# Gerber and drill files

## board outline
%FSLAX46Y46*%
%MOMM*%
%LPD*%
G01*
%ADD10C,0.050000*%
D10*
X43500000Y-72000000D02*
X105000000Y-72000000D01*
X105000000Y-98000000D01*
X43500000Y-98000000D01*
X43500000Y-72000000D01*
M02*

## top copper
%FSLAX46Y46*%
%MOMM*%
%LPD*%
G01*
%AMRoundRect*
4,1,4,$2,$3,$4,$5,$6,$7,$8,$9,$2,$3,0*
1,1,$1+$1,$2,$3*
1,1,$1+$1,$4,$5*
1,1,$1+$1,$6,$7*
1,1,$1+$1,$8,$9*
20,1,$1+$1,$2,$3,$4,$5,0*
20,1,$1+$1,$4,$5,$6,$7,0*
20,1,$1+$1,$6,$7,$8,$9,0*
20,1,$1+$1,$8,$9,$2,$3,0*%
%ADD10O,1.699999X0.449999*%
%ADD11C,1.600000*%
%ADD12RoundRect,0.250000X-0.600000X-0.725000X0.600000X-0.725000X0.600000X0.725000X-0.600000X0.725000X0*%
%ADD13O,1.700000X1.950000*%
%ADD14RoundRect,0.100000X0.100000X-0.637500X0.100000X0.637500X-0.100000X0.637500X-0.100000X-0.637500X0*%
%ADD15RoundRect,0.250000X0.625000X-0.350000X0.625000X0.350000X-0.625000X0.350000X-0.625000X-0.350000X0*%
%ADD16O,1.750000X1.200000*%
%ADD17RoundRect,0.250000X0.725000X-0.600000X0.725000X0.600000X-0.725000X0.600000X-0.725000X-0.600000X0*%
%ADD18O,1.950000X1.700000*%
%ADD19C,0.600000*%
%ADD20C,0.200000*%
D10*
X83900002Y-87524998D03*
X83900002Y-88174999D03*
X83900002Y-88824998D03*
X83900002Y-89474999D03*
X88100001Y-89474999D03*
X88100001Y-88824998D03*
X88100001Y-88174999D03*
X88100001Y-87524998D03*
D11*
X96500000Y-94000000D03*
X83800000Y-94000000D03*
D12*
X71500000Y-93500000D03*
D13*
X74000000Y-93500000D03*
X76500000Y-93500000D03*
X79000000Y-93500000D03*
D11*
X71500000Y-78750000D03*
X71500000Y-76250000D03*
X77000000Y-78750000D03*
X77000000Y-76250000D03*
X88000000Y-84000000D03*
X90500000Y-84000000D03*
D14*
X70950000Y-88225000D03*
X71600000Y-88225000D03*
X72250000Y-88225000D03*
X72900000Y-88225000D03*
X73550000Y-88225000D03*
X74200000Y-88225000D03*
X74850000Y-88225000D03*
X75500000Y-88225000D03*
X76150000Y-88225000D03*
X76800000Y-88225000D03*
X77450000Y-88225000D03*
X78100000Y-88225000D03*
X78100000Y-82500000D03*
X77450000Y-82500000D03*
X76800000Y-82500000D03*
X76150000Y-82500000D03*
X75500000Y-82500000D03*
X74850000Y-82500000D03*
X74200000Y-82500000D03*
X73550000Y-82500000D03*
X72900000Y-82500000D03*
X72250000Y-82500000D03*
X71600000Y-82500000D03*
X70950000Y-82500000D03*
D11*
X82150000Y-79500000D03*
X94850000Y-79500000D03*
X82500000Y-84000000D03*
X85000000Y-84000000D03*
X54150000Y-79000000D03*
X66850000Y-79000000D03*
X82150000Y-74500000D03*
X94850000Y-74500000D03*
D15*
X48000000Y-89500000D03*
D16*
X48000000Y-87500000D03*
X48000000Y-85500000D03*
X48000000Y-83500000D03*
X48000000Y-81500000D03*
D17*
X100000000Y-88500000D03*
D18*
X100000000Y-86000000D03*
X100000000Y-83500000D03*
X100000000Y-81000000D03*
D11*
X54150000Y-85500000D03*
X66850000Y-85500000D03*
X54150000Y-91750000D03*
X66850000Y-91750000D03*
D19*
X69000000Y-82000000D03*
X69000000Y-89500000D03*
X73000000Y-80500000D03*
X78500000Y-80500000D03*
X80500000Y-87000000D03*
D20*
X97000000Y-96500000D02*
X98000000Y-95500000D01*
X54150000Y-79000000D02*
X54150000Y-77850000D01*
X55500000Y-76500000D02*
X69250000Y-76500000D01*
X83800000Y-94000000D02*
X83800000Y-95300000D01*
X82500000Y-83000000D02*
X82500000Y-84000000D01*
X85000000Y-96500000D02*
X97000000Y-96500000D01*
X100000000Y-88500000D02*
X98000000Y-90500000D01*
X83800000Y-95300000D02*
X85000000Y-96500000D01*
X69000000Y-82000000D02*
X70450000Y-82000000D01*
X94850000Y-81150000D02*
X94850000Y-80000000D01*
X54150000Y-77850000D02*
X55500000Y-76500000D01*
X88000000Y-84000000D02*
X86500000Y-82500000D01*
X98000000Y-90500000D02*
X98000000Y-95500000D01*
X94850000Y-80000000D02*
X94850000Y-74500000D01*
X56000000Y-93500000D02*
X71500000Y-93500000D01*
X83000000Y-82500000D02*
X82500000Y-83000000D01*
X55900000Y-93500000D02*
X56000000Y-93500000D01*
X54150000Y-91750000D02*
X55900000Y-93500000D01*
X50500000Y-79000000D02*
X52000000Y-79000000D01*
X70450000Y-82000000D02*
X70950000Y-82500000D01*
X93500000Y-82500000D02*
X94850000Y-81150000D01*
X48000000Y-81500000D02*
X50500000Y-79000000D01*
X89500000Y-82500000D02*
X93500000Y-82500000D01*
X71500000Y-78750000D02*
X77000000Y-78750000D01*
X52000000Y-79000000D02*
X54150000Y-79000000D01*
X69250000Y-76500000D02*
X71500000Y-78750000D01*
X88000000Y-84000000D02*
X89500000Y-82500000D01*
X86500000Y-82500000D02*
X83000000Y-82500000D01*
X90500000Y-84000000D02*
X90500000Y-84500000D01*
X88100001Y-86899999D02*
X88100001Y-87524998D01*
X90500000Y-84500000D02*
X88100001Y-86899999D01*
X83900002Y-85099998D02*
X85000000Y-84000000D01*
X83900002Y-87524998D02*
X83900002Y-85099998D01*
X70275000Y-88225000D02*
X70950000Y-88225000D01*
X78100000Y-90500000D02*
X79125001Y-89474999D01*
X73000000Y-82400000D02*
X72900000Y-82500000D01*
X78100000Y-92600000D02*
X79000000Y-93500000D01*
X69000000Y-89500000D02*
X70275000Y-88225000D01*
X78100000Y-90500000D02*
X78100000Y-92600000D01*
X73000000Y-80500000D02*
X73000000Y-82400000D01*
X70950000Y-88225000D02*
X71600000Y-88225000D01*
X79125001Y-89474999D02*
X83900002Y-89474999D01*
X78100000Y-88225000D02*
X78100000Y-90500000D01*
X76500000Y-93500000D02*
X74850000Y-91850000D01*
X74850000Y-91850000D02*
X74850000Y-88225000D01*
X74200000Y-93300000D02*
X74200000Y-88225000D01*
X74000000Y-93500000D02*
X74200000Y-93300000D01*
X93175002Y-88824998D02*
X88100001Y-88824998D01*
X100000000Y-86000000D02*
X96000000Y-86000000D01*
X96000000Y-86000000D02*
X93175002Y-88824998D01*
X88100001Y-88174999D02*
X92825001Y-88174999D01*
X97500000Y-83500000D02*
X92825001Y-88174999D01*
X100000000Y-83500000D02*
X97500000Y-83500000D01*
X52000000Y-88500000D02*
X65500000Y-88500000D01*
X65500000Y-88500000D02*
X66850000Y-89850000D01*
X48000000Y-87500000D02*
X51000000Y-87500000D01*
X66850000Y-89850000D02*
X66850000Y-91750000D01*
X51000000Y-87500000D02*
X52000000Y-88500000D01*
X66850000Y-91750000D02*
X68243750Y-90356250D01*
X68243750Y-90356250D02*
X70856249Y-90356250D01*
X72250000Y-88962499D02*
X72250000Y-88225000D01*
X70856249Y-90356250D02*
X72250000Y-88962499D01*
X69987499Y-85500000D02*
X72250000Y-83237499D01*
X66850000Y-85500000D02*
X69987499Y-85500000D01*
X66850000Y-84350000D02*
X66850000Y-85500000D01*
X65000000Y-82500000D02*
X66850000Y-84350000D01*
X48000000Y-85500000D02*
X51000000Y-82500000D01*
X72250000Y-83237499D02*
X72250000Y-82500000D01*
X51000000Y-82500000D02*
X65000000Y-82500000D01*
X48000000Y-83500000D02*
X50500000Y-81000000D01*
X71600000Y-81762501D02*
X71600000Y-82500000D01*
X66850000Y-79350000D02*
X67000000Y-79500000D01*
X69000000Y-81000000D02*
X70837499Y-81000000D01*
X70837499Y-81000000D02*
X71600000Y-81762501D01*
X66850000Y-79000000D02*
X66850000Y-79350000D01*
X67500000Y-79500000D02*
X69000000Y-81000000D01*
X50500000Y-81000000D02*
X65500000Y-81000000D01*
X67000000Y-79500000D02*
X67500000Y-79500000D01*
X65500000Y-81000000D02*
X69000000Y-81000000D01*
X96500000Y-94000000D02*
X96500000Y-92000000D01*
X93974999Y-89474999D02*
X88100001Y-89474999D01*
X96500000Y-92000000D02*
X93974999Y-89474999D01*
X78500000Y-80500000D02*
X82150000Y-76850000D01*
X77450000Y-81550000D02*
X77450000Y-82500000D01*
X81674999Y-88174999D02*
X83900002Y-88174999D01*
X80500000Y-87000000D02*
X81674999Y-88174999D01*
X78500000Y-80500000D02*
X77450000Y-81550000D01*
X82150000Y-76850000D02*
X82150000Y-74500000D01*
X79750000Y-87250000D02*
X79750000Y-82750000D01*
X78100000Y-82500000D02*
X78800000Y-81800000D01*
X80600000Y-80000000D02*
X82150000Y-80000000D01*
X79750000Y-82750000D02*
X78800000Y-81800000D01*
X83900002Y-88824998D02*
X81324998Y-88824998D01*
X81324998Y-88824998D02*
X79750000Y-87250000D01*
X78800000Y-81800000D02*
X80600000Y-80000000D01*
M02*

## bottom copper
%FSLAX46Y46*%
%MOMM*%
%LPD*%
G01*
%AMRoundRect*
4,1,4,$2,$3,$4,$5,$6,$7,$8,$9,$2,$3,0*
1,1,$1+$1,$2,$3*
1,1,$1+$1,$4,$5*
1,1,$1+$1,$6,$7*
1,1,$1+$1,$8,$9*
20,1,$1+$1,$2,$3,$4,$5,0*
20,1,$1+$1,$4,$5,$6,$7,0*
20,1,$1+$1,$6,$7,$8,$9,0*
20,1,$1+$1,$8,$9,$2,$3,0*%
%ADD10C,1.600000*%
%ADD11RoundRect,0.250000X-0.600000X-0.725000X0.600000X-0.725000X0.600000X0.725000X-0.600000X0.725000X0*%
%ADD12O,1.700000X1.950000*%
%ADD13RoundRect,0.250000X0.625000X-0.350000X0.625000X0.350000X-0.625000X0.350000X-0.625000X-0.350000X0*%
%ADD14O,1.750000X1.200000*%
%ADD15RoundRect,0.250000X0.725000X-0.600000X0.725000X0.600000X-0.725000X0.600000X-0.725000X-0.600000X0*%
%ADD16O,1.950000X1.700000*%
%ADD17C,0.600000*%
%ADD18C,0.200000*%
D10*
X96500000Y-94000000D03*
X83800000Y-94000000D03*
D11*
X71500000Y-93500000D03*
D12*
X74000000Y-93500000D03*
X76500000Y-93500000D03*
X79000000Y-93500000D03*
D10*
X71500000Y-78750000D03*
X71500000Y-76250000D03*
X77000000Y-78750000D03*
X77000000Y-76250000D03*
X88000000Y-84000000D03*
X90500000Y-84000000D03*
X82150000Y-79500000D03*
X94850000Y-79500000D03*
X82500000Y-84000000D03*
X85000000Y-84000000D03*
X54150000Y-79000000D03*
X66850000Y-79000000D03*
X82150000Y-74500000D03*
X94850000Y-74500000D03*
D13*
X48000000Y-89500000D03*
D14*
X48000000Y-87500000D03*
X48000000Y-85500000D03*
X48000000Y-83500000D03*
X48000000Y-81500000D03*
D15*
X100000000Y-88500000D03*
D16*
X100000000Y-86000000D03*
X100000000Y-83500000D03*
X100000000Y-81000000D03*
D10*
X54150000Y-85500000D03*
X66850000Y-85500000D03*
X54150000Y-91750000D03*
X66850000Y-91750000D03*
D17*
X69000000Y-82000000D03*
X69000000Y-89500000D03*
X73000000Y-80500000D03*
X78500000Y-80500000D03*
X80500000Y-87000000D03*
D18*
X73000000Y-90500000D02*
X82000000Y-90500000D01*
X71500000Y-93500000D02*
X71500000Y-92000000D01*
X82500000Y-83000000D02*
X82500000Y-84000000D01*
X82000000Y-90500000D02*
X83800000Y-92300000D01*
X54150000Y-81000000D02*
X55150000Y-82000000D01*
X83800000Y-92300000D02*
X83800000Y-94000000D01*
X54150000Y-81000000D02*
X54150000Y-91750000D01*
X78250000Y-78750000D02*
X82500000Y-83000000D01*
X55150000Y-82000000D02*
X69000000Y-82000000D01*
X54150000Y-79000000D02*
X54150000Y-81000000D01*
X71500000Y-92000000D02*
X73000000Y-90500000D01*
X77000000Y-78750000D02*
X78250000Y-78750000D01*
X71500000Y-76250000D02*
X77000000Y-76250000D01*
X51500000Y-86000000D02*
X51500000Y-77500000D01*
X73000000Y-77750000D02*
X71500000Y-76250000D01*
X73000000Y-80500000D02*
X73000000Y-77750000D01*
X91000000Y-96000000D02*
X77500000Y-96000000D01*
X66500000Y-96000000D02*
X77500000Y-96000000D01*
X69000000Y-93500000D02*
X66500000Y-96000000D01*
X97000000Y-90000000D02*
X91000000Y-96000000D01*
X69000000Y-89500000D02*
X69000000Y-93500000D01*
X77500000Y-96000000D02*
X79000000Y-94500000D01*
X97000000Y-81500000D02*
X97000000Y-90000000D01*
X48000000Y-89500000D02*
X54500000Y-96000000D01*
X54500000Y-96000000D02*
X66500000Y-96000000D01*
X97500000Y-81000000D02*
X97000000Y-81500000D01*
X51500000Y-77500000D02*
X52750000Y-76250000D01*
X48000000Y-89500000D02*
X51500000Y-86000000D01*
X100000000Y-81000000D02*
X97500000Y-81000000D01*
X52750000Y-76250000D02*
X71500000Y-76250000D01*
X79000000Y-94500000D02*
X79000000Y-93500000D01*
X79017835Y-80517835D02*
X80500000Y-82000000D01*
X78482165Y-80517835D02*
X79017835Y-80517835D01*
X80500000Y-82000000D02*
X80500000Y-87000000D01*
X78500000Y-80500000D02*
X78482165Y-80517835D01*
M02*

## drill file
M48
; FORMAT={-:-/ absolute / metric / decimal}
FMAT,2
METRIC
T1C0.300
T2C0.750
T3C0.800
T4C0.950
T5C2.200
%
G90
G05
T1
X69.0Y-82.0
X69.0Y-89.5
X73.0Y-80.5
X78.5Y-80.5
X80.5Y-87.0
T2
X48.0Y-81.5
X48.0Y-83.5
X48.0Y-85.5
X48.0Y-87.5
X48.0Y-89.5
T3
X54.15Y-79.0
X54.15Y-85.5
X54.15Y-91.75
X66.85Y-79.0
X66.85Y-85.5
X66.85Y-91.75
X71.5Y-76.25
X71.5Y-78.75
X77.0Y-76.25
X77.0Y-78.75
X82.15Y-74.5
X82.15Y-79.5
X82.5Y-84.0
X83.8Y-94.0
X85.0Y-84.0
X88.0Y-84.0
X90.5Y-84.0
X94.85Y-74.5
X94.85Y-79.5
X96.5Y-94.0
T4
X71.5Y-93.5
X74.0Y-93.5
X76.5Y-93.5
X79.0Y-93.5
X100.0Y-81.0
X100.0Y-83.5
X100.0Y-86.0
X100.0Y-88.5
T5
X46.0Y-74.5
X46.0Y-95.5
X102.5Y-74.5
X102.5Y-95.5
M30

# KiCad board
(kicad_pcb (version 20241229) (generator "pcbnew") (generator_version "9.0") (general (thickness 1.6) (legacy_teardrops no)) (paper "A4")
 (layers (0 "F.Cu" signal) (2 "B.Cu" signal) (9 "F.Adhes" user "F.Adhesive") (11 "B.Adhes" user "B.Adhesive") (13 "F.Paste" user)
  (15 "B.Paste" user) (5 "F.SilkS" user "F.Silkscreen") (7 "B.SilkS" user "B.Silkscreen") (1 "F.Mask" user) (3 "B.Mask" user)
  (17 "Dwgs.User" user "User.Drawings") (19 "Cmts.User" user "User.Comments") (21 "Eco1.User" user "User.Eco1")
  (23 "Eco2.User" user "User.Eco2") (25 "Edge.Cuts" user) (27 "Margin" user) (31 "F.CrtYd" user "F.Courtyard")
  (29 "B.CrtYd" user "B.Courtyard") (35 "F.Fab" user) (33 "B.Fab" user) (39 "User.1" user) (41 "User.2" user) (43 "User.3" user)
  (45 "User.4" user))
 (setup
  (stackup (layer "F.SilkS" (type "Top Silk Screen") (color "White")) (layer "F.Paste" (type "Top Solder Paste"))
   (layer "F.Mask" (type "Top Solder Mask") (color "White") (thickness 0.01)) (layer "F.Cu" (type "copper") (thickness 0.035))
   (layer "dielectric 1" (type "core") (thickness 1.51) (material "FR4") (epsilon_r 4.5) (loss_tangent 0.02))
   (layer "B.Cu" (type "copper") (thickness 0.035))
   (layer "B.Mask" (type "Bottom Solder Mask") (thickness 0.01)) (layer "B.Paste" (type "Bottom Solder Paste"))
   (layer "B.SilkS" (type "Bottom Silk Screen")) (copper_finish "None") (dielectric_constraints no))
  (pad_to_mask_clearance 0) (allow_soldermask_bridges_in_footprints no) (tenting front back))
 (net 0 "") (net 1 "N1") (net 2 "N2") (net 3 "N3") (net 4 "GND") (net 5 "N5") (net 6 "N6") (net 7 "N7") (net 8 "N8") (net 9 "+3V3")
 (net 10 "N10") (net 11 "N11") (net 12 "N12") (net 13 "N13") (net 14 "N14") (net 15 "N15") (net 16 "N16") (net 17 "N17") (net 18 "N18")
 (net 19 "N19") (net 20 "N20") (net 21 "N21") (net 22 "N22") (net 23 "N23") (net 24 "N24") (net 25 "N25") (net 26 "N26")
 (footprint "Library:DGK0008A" (layer "F.Cu") (at 86 88.5)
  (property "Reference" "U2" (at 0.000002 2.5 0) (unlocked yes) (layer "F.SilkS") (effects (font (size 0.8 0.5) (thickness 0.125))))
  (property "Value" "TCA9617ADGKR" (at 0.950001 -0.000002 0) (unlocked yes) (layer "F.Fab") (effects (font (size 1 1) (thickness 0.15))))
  (pad "1" smd oval (at -2.099998 -0.975002 90) (size 0.449999 1.699999) (layers "F.Cu" "F.Mask" "F.Paste") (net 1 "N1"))
  (pad "2" smd oval (at -2.099998 -0.325001 90) (size 0.449999 1.699999) (layers "F.Cu" "F.Mask" "F.Paste") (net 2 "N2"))
  (pad "3" smd oval (at -2.099998 0.324998 90) (size 0.449999 1.699999) (layers "F.Cu" "F.Mask" "F.Paste") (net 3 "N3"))
  (pad "4" smd oval (at -2.099998 0.974999 90) (size 0.449999 1.699999) (layers "F.Cu" "F.Mask" "F.Paste") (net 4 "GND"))
  (pad "5" smd oval (at 2.100001 0.974999 90) (size 0.449999 1.699999) (layers "F.Cu" "F.Mask" "F.Paste") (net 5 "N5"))
  (pad "6" smd oval (at 2.100001 0.324998 90) (size 0.449999 1.699999) (layers "F.Cu" "F.Mask" "F.Paste") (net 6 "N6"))
  (pad "7" smd oval (at 2.100001 -0.325001 90) (size 0.449999 1.699999) (layers "F.Cu" "F.Mask" "F.Paste") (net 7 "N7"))
  (pad "8" smd oval (at 2.100001 -0.975002 90) (size 0.449999 1.699999) (layers "F.Cu" "F.Mask" "F.Paste") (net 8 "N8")))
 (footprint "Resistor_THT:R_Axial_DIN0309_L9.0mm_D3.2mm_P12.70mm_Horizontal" (layer "F.Cu") (at 96.5 94 180)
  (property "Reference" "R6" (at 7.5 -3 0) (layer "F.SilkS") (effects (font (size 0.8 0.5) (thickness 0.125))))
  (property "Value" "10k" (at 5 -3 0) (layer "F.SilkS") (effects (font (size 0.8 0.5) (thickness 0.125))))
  (pad "1" thru_hole circle (at 0 0 180) (size 1.6 1.6) (drill 0.8) (layers "*.Cu" "*.Mask") (remove_unused_layers no) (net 5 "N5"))
  (pad "2" thru_hole circle (at 12.7 0 180) (size 1.6 1.6) (drill 0.8) (layers "*.Cu" "*.Mask") (remove_unused_layers no) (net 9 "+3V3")))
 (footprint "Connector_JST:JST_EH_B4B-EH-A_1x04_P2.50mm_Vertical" (layer "F.Cu") (at 71.5 93.5)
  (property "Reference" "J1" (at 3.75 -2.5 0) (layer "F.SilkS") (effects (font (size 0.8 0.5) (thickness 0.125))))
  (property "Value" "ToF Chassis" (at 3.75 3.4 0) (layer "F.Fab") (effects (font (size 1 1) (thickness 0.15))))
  (pad "1" thru_hole roundrect (at 0 0) (size 1.7 1.95) (drill 0.95) (layers "*.Cu" "*.Mask") (remove_unused_layers no)
   (roundrect_rratio 0.147059) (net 9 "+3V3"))
  (pad "2" thru_hole oval (at 2.5 0) (size 1.7 1.95) (drill 0.95) (layers "*.Cu" "*.Mask") (remove_unused_layers no) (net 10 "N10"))
  (pad "3" thru_hole oval (at 5 0) (size 1.7 1.95) (drill 0.95) (layers "*.Cu" "*.Mask") (remove_unused_layers no) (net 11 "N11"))
  (pad "4" thru_hole oval (at 7.5 0) (size 1.7 1.95) (drill 0.95) (layers "*.Cu" "*.Mask") (remove_unused_layers no) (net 4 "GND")))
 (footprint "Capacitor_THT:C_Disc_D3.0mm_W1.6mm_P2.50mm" (layer "F.Cu") (at 71.5 78.75 90)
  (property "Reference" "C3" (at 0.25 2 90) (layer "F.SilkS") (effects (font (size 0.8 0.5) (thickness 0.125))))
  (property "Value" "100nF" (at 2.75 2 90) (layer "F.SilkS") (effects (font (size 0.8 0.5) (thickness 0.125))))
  (pad "1" thru_hole circle (at 0 0 90) (size 1.6 1.6) (drill 0.8) (layers "*.Cu" "*.Mask") (remove_unused_layers no) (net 9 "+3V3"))
  (pad "2" thru_hole circle (at 2.5 0 90) (size 1.6 1.6) (drill 0.8) (layers "*.Cu" "*.Mask") (remove_unused_layers no) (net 4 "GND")))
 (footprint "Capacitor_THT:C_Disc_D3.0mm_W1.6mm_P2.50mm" (layer "F.Cu") (at 77 78.75 90)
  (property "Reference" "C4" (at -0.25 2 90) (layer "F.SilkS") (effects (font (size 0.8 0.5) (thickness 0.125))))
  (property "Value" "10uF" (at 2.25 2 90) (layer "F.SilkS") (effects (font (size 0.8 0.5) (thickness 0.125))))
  (pad "1" thru_hole circle (at 0 0 90) (size 1.6 1.6) (drill 0.8) (layers "*.Cu" "*.Mask") (remove_unused_layers no) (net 9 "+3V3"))
  (pad "2" thru_hole circle (at 2.5 0 90) (size 1.6 1.6) (drill 0.8) (layers "*.Cu" "*.Mask") (remove_unused_layers no) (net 4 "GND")))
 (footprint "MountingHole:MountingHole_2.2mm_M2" (layer "F.Cu") (at 102.5 95.5)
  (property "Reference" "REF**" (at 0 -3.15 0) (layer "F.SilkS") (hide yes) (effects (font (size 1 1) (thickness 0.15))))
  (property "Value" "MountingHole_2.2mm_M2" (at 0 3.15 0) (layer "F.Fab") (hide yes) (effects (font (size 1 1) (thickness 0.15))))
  (pad "" np_thru_hole circle (at 0 0) (size 2.2 2.2) (drill 2.2) (layers "*.Cu" "*.Mask")))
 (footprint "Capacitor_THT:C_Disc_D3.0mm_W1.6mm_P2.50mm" (layer "F.Cu") (at 88 84)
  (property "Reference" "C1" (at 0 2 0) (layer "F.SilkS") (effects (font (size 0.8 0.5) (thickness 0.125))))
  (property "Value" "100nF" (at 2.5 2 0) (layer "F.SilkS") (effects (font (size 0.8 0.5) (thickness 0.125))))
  (pad "1" thru_hole circle (at 0 0) (size 1.6 1.6) (drill 0.8) (layers "*.Cu" "*.Mask") (remove_unused_layers no) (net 9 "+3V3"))
  (pad "2" thru_hole circle (at 2.5 0) (size 1.6 1.6) (drill 0.8) (layers "*.Cu" "*.Mask") (remove_unused_layers no) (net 8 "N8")))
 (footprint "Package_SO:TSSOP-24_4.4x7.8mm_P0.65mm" (layer "F.Cu") (at 74.525 85.3625 90)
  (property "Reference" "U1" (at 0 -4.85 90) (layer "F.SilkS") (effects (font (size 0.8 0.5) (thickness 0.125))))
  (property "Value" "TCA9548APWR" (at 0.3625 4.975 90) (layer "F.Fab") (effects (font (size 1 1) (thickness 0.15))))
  (pad "1" smd roundrect (at -2.8625 -3.575 90) (size 1.475 0.4) (layers "F.Cu" "F.Mask" "F.Paste") (roundrect_rratio 0.25) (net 4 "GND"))
  (pad "2" smd roundrect (at -2.8625 -2.925 90) (size 1.475 0.4) (layers "F.Cu" "F.Mask" "F.Paste") (roundrect_rratio 0.25) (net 4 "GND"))
  (pad "3" smd roundrect (at -2.8625 -2.275 90) (size 1.475 0.4) (layers "F.Cu" "F.Mask" "F.Paste") (roundrect_rratio 0.25) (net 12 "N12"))
  (pad "4" smd roundrect (at -2.8625 -1.625 90) (size 1.475 0.4) (layers "F.Cu" "F.Mask" "F.Paste") (roundrect_rratio 0.25) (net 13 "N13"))
  (pad "5" smd roundrect (at -2.8625 -0.975 90) (size 1.475 0.4) (layers "F.Cu" "F.Mask" "F.Paste") (roundrect_rratio 0.25) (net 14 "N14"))
  (pad "6" smd roundrect (at -2.8625 -0.325 90) (size 1.475 0.4) (layers "F.Cu" "F.Mask" "F.Paste") (roundrect_rratio 0.25) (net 10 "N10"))
  (pad "7" smd roundrect (at -2.8625 0.325 90) (size 1.475 0.4) (layers "F.Cu" "F.Mask" "F.Paste") (roundrect_rratio 0.25) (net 11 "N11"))
  (pad "8" smd roundrect (at -2.8625 0.975 90) (size 1.475 0.4) (layers "F.Cu" "F.Mask" "F.Paste") (roundrect_rratio 0.25) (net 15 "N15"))
  (pad "9" smd roundrect (at -2.8625 1.625 90) (size 1.475 0.4) (layers "F.Cu" "F.Mask" "F.Paste") (roundrect_rratio 0.25) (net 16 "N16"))
  (pad "10" smd roundrect (at -2.8625 2.275 90) (size 1.475 0.4) (layers "F.Cu" "F.Mask" "F.Paste") (roundrect_rratio 0.25) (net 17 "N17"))
  (pad "11" smd roundrect (at -2.8625 2.925 90) (size 1.475 0.4) (layers "F.Cu" "F.Mask" "F.Paste") (roundrect_rratio 0.25) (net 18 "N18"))
  (pad "12" smd roundrect (at -2.8625 3.575 90) (size 1.475 0.4) (layers "F.Cu" "F.Mask" "F.Paste") (roundrect_rratio 0.25) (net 4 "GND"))
  (pad "13" smd roundrect (at 2.8625 3.575 90) (size 1.475 0.4) (layers "F.Cu" "F.Mask" "F.Paste") (roundrect_rratio 0.25) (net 3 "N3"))
  (pad "14" smd roundrect (at 2.8625 2.925 90) (size 1.475 0.4) (layers "F.Cu" "F.Mask" "F.Paste") (roundrect_rratio 0.25) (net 2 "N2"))
  (pad "15" smd roundrect (at 2.8625 2.275 90) (size 1.475 0.4) (layers "F.Cu" "F.Mask" "F.Paste") (roundrect_rratio 0.25) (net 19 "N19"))
  (pad "16" smd roundrect (at 2.8625 1.625 90) (size 1.475 0.4) (layers "F.Cu" "F.Mask" "F.Paste") (roundrect_rratio 0.25) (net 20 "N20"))
  (pad "17" smd roundrect (at 2.8625 0.975 90) (size 1.475 0.4) (layers "F.Cu" "F.Mask" "F.Paste") (roundrect_rratio 0.25) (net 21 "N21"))
  (pad "18" smd roundrect (at 2.8625 0.325 90) (size 1.475 0.4) (layers "F.Cu" "F.Mask" "F.Paste") (roundrect_rratio 0.25) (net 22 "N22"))
  (pad "19" smd roundrect (at 2.8625 -0.325 90) (size 1.475 0.4) (layers "F.Cu" "F.Mask" "F.Paste") (roundrect_rratio 0.25) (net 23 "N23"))
  (pad "20" smd roundrect (at 2.8625 -0.975 90) (size 1.475 0.4) (layers "F.Cu" "F.Mask" "F.Paste") (roundrect_rratio 0.25) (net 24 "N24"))
  (pad "21" smd roundrect (at 2.8625 -1.625 90) (size 1.475 0.4) (layers "F.Cu" "F.Mask" "F.Paste") (roundrect_rratio 0.25) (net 4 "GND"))
  (pad "22" smd roundrect (at 2.8625 -2.275 90) (size 1.475 0.4) (layers "F.Cu" "F.Mask" "F.Paste") (roundrect_rratio 0.25) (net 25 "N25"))
  (pad "23" smd roundrect (at 2.8625 -2.925 90) (size 1.475 0.4) (layers "F.Cu" "F.Mask" "F.Paste") (roundrect_rratio 0.25) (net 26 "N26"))
  (pad "24" smd roundrect (at 2.8625 -3.575 90) (size 1.475 0.4) (layers "F.Cu" "F.Mask" "F.Paste") (roundrect_rratio 0.25) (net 9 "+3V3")))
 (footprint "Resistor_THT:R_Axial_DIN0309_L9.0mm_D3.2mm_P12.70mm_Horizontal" (layer "F.Cu") (at 82.15 79.5)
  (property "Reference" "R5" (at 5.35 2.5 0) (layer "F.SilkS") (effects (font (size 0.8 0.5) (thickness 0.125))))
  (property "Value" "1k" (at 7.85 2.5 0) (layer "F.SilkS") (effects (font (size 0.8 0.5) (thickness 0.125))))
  (pad "1" thru_hole circle (at 0 0) (size 1.6 1.6) (drill 0.8) (layers "*.Cu" "*.Mask") (remove_unused_layers no) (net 3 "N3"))
  (pad "2" thru_hole circle (at 12.7 0) (size 1.6 1.6) (drill 0.8) (layers "*.Cu" "*.Mask") (remove_unused_layers no) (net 9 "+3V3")))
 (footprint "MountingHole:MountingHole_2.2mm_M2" (layer "F.Cu") (at 46 74.5)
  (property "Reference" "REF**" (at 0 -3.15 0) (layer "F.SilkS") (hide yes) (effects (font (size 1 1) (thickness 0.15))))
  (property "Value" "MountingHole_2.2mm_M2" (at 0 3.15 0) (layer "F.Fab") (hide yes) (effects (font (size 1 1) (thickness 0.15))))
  (pad "" np_thru_hole circle (at 0 0) (size 2.2 2.2) (drill 2.2) (layers "*.Cu" "*.Mask")))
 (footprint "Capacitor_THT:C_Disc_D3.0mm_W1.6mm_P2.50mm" (layer "F.Cu") (at 82.5 84)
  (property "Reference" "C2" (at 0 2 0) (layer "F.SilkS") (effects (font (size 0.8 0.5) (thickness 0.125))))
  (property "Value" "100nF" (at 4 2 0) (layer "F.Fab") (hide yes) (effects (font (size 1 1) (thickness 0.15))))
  (pad "1" thru_hole circle (at 0 0) (size 1.6 1.6) (drill 0.8) (layers "*.Cu" "*.Mask") (remove_unused_layers no) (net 9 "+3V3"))
  (pad "2" thru_hole circle (at 2.5 0) (size 1.6 1.6) (drill 0.8) (layers "*.Cu" "*.Mask") (remove_unused_layers no) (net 1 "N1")))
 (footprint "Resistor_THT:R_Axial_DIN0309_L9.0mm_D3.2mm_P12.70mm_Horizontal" (layer "F.Cu") (at 54.15 79)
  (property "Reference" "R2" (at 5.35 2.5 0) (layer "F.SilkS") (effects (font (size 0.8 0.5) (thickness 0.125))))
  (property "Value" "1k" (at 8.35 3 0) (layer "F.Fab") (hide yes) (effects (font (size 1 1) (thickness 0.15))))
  (pad "1" thru_hole circle (at 0 0) (size 1.6 1.6) (drill 0.8) (layers "*.Cu" "*.Mask") (remove_unused_layers no) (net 9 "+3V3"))
  (pad "2" thru_hole circle (at 12.7 0) (size 1.6 1.6) (drill 0.8) (layers "*.Cu" "*.Mask") (remove_unused_layers no) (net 26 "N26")))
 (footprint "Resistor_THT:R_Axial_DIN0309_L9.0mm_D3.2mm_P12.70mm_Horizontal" (layer "F.Cu") (at 82.15 74.5)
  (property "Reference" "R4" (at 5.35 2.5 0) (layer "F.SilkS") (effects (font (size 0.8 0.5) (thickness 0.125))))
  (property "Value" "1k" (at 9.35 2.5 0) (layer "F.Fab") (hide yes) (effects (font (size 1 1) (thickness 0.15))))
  (pad "1" thru_hole circle (at 0 0) (size 1.6 1.6) (drill 0.8) (layers "*.Cu" "*.Mask") (remove_unused_layers no) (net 2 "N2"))
  (pad "2" thru_hole circle (at 12.7 0) (size 1.6 1.6) (drill 0.8) (layers "*.Cu" "*.Mask") (remove_unused_layers no) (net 9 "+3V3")))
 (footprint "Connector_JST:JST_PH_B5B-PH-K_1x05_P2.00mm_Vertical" (layer "F.Cu") (at 48 89.5 90)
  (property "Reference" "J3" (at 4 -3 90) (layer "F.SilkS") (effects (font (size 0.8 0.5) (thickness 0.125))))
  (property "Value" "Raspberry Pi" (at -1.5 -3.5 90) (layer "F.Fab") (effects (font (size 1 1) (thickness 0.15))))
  (pad "1" thru_hole roundrect (at 0 0 90) (size 1.2 1.75) (drill 0.75) (layers "*.Cu" "*.Mask") (remove_unused_layers no)
   (roundrect_rratio 0.208333) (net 4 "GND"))
  (pad "2" thru_hole oval (at 2 0 90) (size 1.2 1.75) (drill 0.75) (layers "*.Cu" "*.Mask") (remove_unused_layers no) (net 12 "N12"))
  (pad "3" thru_hole oval (at 4 0 90) (size 1.2 1.75) (drill 0.75) (layers "*.Cu" "*.Mask") (remove_unused_layers no) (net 25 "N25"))
  (pad "4" thru_hole oval (at 6 0 90) (size 1.2 1.75) (drill 0.75) (layers "*.Cu" "*.Mask") (remove_unused_layers no) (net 26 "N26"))
  (pad "5" thru_hole oval (at 8 0 90) (size 1.2 1.75) (drill 0.75) (layers "*.Cu" "*.Mask") (remove_unused_layers no) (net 9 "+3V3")))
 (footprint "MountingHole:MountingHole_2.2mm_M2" (layer "F.Cu") (at 102.5 74.5)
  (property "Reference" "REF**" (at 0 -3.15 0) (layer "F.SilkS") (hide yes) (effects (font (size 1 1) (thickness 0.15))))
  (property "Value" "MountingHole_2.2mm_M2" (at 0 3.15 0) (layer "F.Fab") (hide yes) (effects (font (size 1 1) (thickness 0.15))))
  (pad "" np_thru_hole circle (at 0 0) (size 2.2 2.2) (drill 2.2) (layers "*.Cu" "*.Mask")))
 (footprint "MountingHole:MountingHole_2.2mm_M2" (layer "F.Cu") (at 46 95.5)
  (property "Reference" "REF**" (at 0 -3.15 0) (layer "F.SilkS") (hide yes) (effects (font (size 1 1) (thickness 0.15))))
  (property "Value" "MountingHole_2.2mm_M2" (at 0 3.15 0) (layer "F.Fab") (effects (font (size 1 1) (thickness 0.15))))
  (pad "" np_thru_hole circle (at 0 0) (size 2.2 2.2) (drill 2.2) (layers "*.Cu" "*.Mask")))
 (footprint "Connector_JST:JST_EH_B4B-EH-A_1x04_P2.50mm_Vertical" (layer "F.Cu") (at 100 88.5 90)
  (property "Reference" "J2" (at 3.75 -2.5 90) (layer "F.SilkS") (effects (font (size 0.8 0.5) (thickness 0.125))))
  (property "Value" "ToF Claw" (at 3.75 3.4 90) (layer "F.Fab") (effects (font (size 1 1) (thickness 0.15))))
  (pad "1" thru_hole roundrect (at 0 0 90) (size 1.7 1.95) (drill 0.95) (layers "*.Cu" "*.Mask") (remove_unused_layers no)
   (roundrect_rratio 0.147059) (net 9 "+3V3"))
  (pad "2" thru_hole oval (at 2.5 0 90) (size 1.7 1.95) (drill 0.95) (layers "*.Cu" "*.Mask") (remove_unused_layers no) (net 6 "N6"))
  (pad "3" thru_hole oval (at 5 0 90) (size 1.7 1.95) (drill 0.95) (layers "*.Cu" "*.Mask") (remove_unused_layers no) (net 7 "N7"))
  (pad "4" thru_hole oval (at 7.5 0 90) (size 1.7 1.95) (drill 0.95) (layers "*.Cu" "*.Mask") (remove_unused_layers no) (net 4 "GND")))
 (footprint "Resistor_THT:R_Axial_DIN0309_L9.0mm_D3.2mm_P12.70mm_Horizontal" (layer "F.Cu") (at 54.15 85.5)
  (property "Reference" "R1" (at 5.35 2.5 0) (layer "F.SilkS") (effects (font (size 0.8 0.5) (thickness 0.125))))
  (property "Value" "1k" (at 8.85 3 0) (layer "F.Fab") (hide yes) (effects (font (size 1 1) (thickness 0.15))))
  (pad "1" thru_hole circle (at 0 0) (size 1.6 1.6) (drill 0.8) (layers "*.Cu" "*.Mask") (remove_unused_layers no) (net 9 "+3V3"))
  (pad "2" thru_hole circle (at 12.7 0) (size 1.6 1.6) (drill 0.8) (layers "*.Cu" "*.Mask") (remove_unused_layers no) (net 25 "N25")))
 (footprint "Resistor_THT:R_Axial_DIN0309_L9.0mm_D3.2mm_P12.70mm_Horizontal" (layer "F.Cu") (at 54.15 91.75)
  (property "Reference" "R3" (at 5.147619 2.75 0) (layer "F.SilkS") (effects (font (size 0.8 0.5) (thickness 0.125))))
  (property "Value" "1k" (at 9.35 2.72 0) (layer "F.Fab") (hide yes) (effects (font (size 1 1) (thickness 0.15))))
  (pad "1" thru_hole circle (at 0 0) (size 1.6 1.6) (drill 0.8) (layers "*.Cu" "*.Mask") (remove_unused_layers no) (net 9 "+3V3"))
  (pad "2" thru_hole circle (at 12.7 0) (size 1.6 1.6) (drill 0.8) (layers "*.Cu" "*.Mask") (remove_unused_layers no) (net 12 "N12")))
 (gr_rect (start 43.5 72) (end 105 98) (stroke (width 0.05) (type default)) (fill no) (layer "Edge.Cuts"))
 (segment (start 97 96.5) (end 98 95.5) (width 0.2) (layer "F.Cu") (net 9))
 (segment (start 54.15 79) (end 54.15 77.85) (width 0.2) (layer "F.Cu") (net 9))
 (segment (start 55.5 76.5) (end 69.25 76.5) (width 0.2) (layer "F.Cu") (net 9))
 (segment (start 83.8 94) (end 83.8 95.3) (width 0.2) (layer "F.Cu") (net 9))
 (segment (start 82.5 83) (end 82.5 84) (width 0.2) (layer "F.Cu") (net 9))
 (segment (start 85 96.5) (end 97 96.5) (width 0.2) (layer "F.Cu") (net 9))
 (segment (start 100 88.5) (end 98 90.5) (width 0.2) (layer "F.Cu") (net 9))
 (segment (start 83.8 95.3) (end 85 96.5) (width 0.2) (layer "F.Cu") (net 9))
 (segment (start 69 82) (end 70.45 82) (width 0.2) (layer "F.Cu") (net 9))
 (segment (start 94.85 81.15) (end 94.85 80) (width 0.2) (layer "F.Cu") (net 9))
 (segment (start 54.15 77.85) (end 55.5 76.5) (width 0.2) (layer "F.Cu") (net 9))
 (segment (start 88 84) (end 86.5 82.5) (width 0.2) (layer "F.Cu") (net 9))
 (segment (start 98 90.5) (end 98 95.5) (width 0.2) (layer "F.Cu") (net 9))
 (segment (start 94.85 80) (end 94.85 74.5) (width 0.2) (layer "F.Cu") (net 9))
 (segment (start 56 93.5) (end 71.5 93.5) (width 0.2) (layer "F.Cu") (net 9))
 (segment (start 83 82.5) (end 82.5 83) (width 0.2) (layer "F.Cu") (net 9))
 (segment (start 55.9 93.5) (end 56 93.5) (width 0.2) (layer "F.Cu") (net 9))
 (segment (start 54.15 91.75) (end 55.9 93.5) (width 0.2) (layer "F.Cu") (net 9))
 (segment (start 50.5 79) (end 52 79) (width 0.2) (layer "F.Cu") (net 9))
 (segment (start 70.45 82) (end 70.95 82.5) (width 0.2) (layer "F.Cu") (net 9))
 (segment (start 93.5 82.5) (end 94.85 81.15) (width 0.2) (layer "F.Cu") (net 9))
 (segment (start 48 81.5) (end 50.5 79) (width 0.2) (layer "F.Cu") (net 9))
 (segment (start 89.5 82.5) (end 93.5 82.5) (width 0.2) (layer "F.Cu") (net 9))
 (segment (start 71.5 78.75) (end 77 78.75) (width 0.2) (layer "F.Cu") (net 9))
 (segment (start 52 79) (end 54.15 79) (width 0.2) (layer "F.Cu") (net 9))
 (segment (start 69.25 76.5) (end 71.5 78.75) (width 0.2) (layer "F.Cu") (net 9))
 (segment (start 88 84) (end 89.5 82.5) (width 0.2) (layer "F.Cu") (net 9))
 (segment (start 86.5 82.5) (end 83 82.5) (width 0.2) (layer "F.Cu") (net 9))
 (via (at 69 82) (size 0.6) (drill 0.3) (layers "F.Cu" "B.Cu") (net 9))
 (segment (start 73 90.5) (end 82 90.5) (width 0.2) (layer "B.Cu") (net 9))
 (segment (start 71.5 93.5) (end 71.5 92) (width 0.2) (layer "B.Cu") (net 9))
 (segment (start 82.5 83) (end 82.5 84) (width 0.2) (layer "B.Cu") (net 9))
 (segment (start 82 90.5) (end 83.8 92.3) (width 0.2) (layer "B.Cu") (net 9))
 (segment (start 54.15 81) (end 55.15 82) (width 0.2) (layer "B.Cu") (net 9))
 (segment (start 83.8 92.3) (end 83.8 94) (width 0.2) (layer "B.Cu") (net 9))
 (segment (start 54.15 81) (end 54.15 91.75) (width 0.2) (layer "B.Cu") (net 9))
 (segment (start 78.25 78.75) (end 82.5 83) (width 0.2) (layer "B.Cu") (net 9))
 (segment (start 55.15 82) (end 69 82) (width 0.2) (layer "B.Cu") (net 9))
 (segment (start 54.15 79) (end 54.15 81) (width 0.2) (layer "B.Cu") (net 9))
 (segment (start 71.5 92) (end 73 90.5) (width 0.2) (layer "B.Cu") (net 9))
 (segment (start 77 78.75) (end 78.25 78.75) (width 0.2) (layer "B.Cu") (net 9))
 (segment (start 90.5 84) (end 90.5 84.5) (width 0.2) (layer "F.Cu") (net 8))
 (segment (start 88.100001 86.899999) (end 88.100001 87.524998) (width 0.2) (layer "F.Cu") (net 8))
 (segment (start 90.5 84.5) (end 88.100001 86.899999) (width 0.2) (layer "F.Cu") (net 8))
 (segment (start 83.900002 85.099998) (end 85 84) (width 0.2) (layer "F.Cu") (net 1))
 (segment (start 83.900002 87.524998) (end 83.900002 85.099998) (width 0.2) (layer "F.Cu") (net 1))
 (segment (start 70.275 88.225) (end 70.95 88.225) (width 0.2) (layer "F.Cu") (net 4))
 (segment (start 78.1 90.5) (end 79.125001 89.474999) (width 0.2) (layer "F.Cu") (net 4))
 (segment (start 73 82.4) (end 72.9 82.5) (width 0.2) (layer "F.Cu") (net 4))
 (segment (start 78.1 92.6) (end 79 93.5) (width 0.2) (layer "F.Cu") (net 4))
 (segment (start 69 89.5) (end 70.275 88.225) (width 0.2) (layer "F.Cu") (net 4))
 (segment (start 78.1 90.5) (end 78.1 92.6) (width 0.2) (layer "F.Cu") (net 4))
 (segment (start 73 80.5) (end 73 82.4) (width 0.2) (layer "F.Cu") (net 4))
 (segment (start 70.95 88.225) (end 71.6 88.225) (width 0.2) (layer "F.Cu") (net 4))
 (segment (start 79.125001 89.474999) (end 83.900002 89.474999) (width 0.2) (layer "F.Cu") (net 4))
 (segment (start 78.1 88.225) (end 78.1 90.5) (width 0.2) (layer "F.Cu") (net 4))
 (via (at 69 89.5) (size 0.6) (drill 0.3) (layers "F.Cu" "B.Cu") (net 4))
 (via (at 73 80.5) (size 0.6) (drill 0.3) (layers "F.Cu" "B.Cu") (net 4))
 (segment (start 71.5 76.25) (end 77 76.25) (width 0.2) (layer "B.Cu") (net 4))
 (segment (start 51.5 86) (end 51.5 77.5) (width 0.2) (layer "B.Cu") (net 4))
 (segment (start 73 77.75) (end 71.5 76.25) (width 0.2) (layer "B.Cu") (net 4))
 (segment (start 73 80.5) (end 73 77.75) (width 0.2) (layer "B.Cu") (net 4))
 (segment (start 91 96) (end 77.5 96) (width 0.2) (layer "B.Cu") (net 4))
 (segment (start 66.5 96) (end 77.5 96) (width 0.2) (layer "B.Cu") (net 4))
 (segment (start 69 93.5) (end 66.5 96) (width 0.2) (layer "B.Cu") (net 4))
 (segment (start 97 90) (end 91 96) (width 0.2) (layer "B.Cu") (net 4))
 (segment (start 69 89.5) (end 69 93.5) (width 0.2) (layer "B.Cu") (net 4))
 (segment (start 77.5 96) (end 79 94.5) (width 0.2) (layer "B.Cu") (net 4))
 (segment (start 97 81.5) (end 97 90) (width 0.2) (layer "B.Cu") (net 4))
 (segment (start 48 89.5) (end 54.5 96) (width 0.2) (layer "B.Cu") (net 4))
 (segment (start 54.5 96) (end 66.5 96) (width 0.2) (layer "B.Cu") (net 4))
 (segment (start 97.5 81) (end 97 81.5) (width 0.2) (layer "B.Cu") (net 4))
 (segment (start 51.5 77.5) (end 52.75 76.25) (width 0.2) (layer "B.Cu") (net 4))
 (segment (start 48 89.5) (end 51.5 86) (width 0.2) (layer "B.Cu") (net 4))
 (segment (start 100 81) (end 97.5 81) (width 0.2) (layer "B.Cu") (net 4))
 (segment (start 52.75 76.25) (end 71.5 76.25) (width 0.2) (layer "B.Cu") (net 4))
 (segment (start 79 94.5) (end 79 93.5) (width 0.2) (layer "B.Cu") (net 4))
 (segment (start 76.5 93.5) (end 74.85 91.85) (width 0.2) (layer "F.Cu") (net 11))
 (segment (start 74.85 91.85) (end 74.85 88.225) (width 0.2) (layer "F.Cu") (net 11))
 (segment (start 74.2 93.3) (end 74.2 88.225) (width 0.2) (layer "F.Cu") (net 10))
 (segment (start 74 93.5) (end 74.2 93.3) (width 0.2) (layer "F.Cu") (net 10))
 (segment (start 93.175002 88.824998) (end 88.100001 88.824998) (width 0.2) (layer "F.Cu") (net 6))
 (segment (start 100 86) (end 96 86) (width 0.2) (layer "F.Cu") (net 6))
 (segment (start 96 86) (end 93.175002 88.824998) (width 0.2) (layer "F.Cu") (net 6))
 (segment (start 88.100001 88.174999) (end 92.825001 88.174999) (width 0.2) (layer "F.Cu") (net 7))
 (segment (start 97.5 83.5) (end 92.825001 88.174999) (width 0.2) (layer "F.Cu") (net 7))
 (segment (start 100 83.5) (end 97.5 83.5) (width 0.2) (layer "F.Cu") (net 7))
 (segment (start 52 88.5) (end 65.5 88.5) (width 0.2) (layer "F.Cu") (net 12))
 (segment (start 65.5 88.5) (end 66.85 89.85) (width 0.2) (layer "F.Cu") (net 12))
 (segment (start 48 87.5) (end 51 87.5) (width 0.2) (layer "F.Cu") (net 12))
 (segment (start 66.85 89.85) (end 66.85 91.75) (width 0.2) (layer "F.Cu") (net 12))
 (segment (start 51 87.5) (end 52 88.5) (width 0.2) (layer "F.Cu") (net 12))
 (segment (start 66.85 91.75) (end 68.24375 90.35625) (width 0.2) (layer "F.Cu") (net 12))
 (segment (start 68.24375 90.35625) (end 70.856249 90.35625) (width 0.2) (layer "F.Cu") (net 12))
 (segment (start 72.25 88.962499) (end 72.25 88.225) (width 0.2) (layer "F.Cu") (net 12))
 (segment (start 70.856249 90.35625) (end 72.25 88.962499) (width 0.2) (layer "F.Cu") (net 12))
 (segment (start 69.987499 85.5) (end 72.25 83.237499) (width 0.2) (layer "F.Cu") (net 25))
 (segment (start 66.85 85.5) (end 69.987499 85.5) (width 0.2) (layer "F.Cu") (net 25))
 (segment (start 66.85 84.35) (end 66.85 85.5) (width 0.2) (layer "F.Cu") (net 25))
 (segment (start 65 82.5) (end 66.85 84.35) (width 0.2) (layer "F.Cu") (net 25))
 (segment (start 48 85.5) (end 51 82.5) (width 0.2) (layer "F.Cu") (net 25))
 (segment (start 72.25 83.237499) (end 72.25 82.5) (width 0.2) (layer "F.Cu") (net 25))
 (segment (start 51 82.5) (end 65 82.5) (width 0.2) (layer "F.Cu") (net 25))
 (segment (start 48 83.5) (end 50.5 81) (width 0.2) (layer "F.Cu") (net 26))
 (segment (start 71.6 81.762501) (end 71.6 82.5) (width 0.2) (layer "F.Cu") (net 26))
 (segment (start 66.85 79.35) (end 67 79.5) (width 0.2) (layer "F.Cu") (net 26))
 (segment (start 69 81) (end 70.837499 81) (width 0.2) (layer "F.Cu") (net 26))
 (segment (start 70.837499 81) (end 71.6 81.762501) (width 0.2) (layer "F.Cu") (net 26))
 (segment (start 66.85 79) (end 66.85 79.35) (width 0.2) (layer "F.Cu") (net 26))
 (segment (start 67.5 79.5) (end 69 81) (width 0.2) (layer "F.Cu") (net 26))
 (segment (start 50.5 81) (end 65.5 81) (width 0.2) (layer "F.Cu") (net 26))
 (segment (start 67 79.5) (end 67.5 79.5) (width 0.2) (layer "F.Cu") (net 26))
 (segment (start 65.5 81) (end 69 81) (width 0.2) (layer "F.Cu") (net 26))
 (segment (start 96.5 94) (end 96.5 92) (width 0.2) (layer "F.Cu") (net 5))
 (segment (start 93.974999 89.474999) (end 88.100001 89.474999) (width 0.2) (layer "F.Cu") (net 5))
 (segment (start 96.5 92) (end 93.974999 89.474999) (width 0.2) (layer "F.Cu") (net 5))
 (segment (start 78.5 80.5) (end 82.15 76.85) (width 0.2) (layer "F.Cu") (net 2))
 (segment (start 77.45 81.55) (end 77.45 82.5) (width 0.2) (layer "F.Cu") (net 2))
 (segment (start 81.674999 88.174999) (end 83.900002 88.174999) (width 0.2) (layer "F.Cu") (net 2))
 (segment (start 80.5 87) (end 81.674999 88.174999) (width 0.2) (layer "F.Cu") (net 2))
 (segment (start 78.5 80.5) (end 77.45 81.55) (width 0.2) (layer "F.Cu") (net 2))
 (segment (start 82.15 76.85) (end 82.15 74.5) (width 0.2) (layer "F.Cu") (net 2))
 (via (at 78.5 80.5) (size 0.6) (drill 0.3) (layers "F.Cu" "B.Cu") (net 2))
 (via (at 80.5 87) (size 0.6) (drill 0.3) (layers "F.Cu" "B.Cu") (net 2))
 (segment (start 79.017835 80.517835) (end 80.5 82) (width 0.2) (layer "B.Cu") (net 2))
 (segment (start 78.482165 80.517835) (end 79.017835 80.517835) (width 0.2) (layer "B.Cu") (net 2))
 (segment (start 80.5 82) (end 80.5 87) (width 0.2) (layer "B.Cu") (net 2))
 (segment (start 78.5 80.5) (end 78.482165 80.517835) (width 0.2) (layer "B.Cu") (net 2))
 (segment (start 79.75 87.25) (end 79.75 82.75) (width 0.2) (layer "F.Cu") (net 3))
 (segment (start 78.1 82.5) (end 78.8 81.8) (width 0.2) (layer "F.Cu") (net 3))
 (segment (start 80.6 80) (end 82.15 80) (width 0.2) (layer "F.Cu") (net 3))
 (segment (start 79.75 82.75) (end 78.8 81.8) (width 0.2) (layer "F.Cu") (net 3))
 (segment (start 83.900002 88.824998) (end 81.324998 88.824998) (width 0.2) (layer "F.Cu") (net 3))
 (segment (start 81.324998 88.824998) (end 79.75 87.25) (width 0.2) (layer "F.Cu") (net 3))
 (segment (start 78.8 81.8) (end 80.6 80) (width 0.2) (layer "F.Cu") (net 3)))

